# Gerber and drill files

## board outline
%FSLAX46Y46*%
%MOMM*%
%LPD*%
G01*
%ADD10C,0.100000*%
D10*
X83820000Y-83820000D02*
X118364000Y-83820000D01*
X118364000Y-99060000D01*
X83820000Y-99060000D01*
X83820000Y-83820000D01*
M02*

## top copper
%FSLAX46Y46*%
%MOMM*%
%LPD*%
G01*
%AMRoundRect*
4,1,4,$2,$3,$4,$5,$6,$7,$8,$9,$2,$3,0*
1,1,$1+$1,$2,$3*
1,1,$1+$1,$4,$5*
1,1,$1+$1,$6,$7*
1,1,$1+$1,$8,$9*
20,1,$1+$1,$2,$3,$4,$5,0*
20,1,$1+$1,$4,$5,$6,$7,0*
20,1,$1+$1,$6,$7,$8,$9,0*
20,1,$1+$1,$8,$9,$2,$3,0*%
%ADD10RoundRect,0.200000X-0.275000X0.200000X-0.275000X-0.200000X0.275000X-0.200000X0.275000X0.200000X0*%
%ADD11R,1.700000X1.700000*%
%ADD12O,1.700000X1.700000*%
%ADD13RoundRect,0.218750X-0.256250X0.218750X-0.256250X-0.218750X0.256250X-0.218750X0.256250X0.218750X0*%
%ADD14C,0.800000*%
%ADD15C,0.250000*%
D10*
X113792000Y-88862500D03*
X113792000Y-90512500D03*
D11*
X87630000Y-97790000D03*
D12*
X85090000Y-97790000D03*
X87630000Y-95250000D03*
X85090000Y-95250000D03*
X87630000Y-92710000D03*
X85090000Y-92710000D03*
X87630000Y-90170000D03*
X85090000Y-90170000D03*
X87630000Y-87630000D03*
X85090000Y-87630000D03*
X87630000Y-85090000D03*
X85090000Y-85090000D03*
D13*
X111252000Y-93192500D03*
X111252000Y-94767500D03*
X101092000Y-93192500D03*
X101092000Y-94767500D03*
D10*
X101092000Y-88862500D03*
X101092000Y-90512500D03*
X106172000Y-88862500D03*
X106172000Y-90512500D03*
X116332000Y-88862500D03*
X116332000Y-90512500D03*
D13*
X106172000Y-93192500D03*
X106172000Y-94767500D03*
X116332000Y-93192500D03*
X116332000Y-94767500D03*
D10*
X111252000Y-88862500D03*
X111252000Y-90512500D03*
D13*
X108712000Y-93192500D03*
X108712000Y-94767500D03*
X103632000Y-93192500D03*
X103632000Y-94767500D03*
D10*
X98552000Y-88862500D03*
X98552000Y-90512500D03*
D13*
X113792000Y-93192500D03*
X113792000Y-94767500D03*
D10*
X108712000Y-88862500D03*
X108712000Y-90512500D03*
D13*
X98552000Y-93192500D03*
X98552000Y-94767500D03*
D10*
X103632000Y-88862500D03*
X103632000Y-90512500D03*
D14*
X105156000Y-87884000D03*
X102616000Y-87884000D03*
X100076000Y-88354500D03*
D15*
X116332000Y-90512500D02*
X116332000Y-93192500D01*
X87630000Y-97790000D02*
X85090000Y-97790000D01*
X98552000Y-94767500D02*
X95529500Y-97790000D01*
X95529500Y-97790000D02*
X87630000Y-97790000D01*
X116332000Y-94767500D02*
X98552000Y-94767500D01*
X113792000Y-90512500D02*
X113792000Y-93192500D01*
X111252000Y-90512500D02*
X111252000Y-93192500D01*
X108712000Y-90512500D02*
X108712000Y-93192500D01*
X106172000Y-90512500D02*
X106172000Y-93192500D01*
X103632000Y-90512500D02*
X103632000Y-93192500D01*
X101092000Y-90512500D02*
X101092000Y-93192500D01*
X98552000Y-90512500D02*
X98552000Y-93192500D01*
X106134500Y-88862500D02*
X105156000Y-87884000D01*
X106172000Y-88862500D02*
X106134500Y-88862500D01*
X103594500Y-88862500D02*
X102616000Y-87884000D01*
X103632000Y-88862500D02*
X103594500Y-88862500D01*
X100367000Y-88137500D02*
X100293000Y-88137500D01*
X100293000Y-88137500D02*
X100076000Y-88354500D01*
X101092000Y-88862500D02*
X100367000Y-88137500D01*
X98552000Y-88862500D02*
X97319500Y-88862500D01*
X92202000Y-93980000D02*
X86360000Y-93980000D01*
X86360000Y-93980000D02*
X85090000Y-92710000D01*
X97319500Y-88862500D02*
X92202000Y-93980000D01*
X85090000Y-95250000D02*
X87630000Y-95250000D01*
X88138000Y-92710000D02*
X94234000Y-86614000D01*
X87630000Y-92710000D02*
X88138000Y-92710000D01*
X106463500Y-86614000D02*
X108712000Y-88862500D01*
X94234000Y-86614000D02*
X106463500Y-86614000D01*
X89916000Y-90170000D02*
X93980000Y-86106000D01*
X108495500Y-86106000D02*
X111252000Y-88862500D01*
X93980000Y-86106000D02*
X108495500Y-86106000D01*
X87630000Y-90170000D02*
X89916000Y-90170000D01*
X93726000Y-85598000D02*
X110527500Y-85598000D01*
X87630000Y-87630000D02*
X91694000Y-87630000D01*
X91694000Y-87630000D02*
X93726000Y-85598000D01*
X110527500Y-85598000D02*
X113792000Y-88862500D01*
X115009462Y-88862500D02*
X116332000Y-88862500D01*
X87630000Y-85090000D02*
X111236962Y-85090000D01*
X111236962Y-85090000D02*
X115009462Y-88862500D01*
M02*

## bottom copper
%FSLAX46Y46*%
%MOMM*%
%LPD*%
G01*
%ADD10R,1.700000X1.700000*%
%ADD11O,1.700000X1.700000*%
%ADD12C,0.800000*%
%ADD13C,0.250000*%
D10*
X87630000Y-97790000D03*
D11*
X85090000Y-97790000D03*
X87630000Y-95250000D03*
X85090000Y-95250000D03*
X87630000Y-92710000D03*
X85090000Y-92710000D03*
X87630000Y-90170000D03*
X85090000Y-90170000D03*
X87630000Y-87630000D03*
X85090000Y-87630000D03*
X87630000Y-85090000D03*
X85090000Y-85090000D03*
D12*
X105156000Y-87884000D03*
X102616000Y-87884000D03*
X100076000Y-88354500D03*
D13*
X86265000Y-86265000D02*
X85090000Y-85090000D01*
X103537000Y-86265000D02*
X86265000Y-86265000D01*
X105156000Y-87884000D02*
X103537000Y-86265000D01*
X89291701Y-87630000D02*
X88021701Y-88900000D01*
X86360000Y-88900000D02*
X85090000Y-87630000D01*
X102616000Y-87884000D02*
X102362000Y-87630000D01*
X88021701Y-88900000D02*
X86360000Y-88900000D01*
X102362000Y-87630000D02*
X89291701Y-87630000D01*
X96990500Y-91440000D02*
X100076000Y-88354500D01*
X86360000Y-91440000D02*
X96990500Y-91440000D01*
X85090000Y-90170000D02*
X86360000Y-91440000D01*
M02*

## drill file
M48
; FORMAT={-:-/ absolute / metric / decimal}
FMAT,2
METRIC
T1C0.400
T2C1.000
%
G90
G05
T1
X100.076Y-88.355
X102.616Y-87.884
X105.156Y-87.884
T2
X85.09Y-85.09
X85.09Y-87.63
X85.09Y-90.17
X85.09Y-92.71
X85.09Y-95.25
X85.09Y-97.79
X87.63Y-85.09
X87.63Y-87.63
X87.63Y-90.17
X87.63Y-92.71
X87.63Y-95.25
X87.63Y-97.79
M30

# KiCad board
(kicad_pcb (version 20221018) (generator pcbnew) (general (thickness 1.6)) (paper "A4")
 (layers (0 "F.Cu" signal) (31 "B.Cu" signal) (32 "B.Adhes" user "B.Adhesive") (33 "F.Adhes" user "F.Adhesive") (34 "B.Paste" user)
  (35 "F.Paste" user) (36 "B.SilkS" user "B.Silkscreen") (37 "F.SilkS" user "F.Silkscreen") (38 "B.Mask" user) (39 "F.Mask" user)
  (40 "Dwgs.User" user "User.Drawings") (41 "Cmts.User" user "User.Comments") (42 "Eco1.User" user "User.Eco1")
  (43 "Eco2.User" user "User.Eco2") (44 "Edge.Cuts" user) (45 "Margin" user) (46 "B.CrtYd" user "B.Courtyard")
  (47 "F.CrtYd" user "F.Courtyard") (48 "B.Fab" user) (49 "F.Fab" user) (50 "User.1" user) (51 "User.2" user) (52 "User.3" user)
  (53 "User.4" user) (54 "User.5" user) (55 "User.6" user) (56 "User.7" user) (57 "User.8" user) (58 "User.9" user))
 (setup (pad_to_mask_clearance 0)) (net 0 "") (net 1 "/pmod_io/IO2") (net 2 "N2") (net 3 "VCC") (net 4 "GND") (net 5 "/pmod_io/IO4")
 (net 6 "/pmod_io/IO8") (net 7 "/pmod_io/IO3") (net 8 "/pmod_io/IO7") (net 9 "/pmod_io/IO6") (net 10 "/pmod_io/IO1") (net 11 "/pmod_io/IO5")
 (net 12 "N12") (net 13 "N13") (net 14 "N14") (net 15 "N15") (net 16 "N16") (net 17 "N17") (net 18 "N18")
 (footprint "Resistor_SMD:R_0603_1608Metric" (layer "F.Cu") (at 113.792 89.6875 -90)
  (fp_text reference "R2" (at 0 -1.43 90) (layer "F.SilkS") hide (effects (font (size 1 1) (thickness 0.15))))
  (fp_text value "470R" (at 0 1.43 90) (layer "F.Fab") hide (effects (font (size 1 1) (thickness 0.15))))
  (pad "1" smd roundrect (at -0.825 0 270) (size 0.8 0.95) (layers "F.Cu" "F.Paste" "F.Mask") (roundrect_rratio 0.25) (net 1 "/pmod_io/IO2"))
  (pad "2" smd roundrect (at 0.825 0 270) (size 0.8 0.95) (layers "F.Cu" "F.Paste" "F.Mask") (roundrect_rratio 0.25) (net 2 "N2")))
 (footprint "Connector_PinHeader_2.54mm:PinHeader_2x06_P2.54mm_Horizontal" (layer "F.Cu") (at 87.63 97.79 180)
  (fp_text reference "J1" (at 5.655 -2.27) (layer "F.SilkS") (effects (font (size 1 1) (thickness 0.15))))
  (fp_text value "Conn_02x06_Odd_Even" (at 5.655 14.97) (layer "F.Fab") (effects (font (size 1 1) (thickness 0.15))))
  (pad "1" thru_hole rect (at 0 0 180) (size 1.7 1.7) (drill 1) (layers "*.Cu" "*.Mask") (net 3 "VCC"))
  (pad "2" thru_hole oval (at 2.54 0 180) (size 1.7 1.7) (drill 1) (layers "*.Cu" "*.Mask") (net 3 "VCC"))
  (pad "3" thru_hole oval (at 0 2.54 180) (size 1.7 1.7) (drill 1) (layers "*.Cu" "*.Mask") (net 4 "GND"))
  (pad "4" thru_hole oval (at 2.54 2.54 180) (size 1.7 1.7) (drill 1) (layers "*.Cu" "*.Mask") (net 4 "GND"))
  (pad "5" thru_hole oval (at 0 5.08 180) (size 1.7 1.7) (drill 1) (layers "*.Cu" "*.Mask") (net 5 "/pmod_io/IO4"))
  (pad "6" thru_hole oval (at 2.54 5.08 180) (size 1.7 1.7) (drill 1) (layers "*.Cu" "*.Mask") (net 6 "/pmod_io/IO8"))
  (pad "7" thru_hole oval (at 0 7.62 180) (size 1.7 1.7) (drill 1) (layers "*.Cu" "*.Mask") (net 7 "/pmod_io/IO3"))
  (pad "8" thru_hole oval (at 2.54 7.62 180) (size 1.7 1.7) (drill 1) (layers "*.Cu" "*.Mask") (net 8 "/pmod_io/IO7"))
  (pad "9" thru_hole oval (at 0 10.16 180) (size 1.7 1.7) (drill 1) (layers "*.Cu" "*.Mask") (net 1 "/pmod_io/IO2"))
  (pad "10" thru_hole oval (at 2.54 10.16 180) (size 1.7 1.7) (drill 1) (layers "*.Cu" "*.Mask") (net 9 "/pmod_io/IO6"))
  (pad "11" thru_hole oval (at 0 12.7 180) (size 1.7 1.7) (drill 1) (layers "*.Cu" "*.Mask") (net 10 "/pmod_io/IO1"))
  (pad "12" thru_hole oval (at 2.54 12.7 180) (size 1.7 1.7) (drill 1) (layers "*.Cu" "*.Mask") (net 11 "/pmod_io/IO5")))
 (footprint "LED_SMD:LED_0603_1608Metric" (layer "F.Cu") (at 111.252 93.98 -90)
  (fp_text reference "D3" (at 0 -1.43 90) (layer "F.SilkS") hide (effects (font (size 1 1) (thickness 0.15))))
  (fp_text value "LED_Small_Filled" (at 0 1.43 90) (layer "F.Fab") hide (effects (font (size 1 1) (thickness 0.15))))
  (pad "1" smd roundrect (at -0.7875 0 270) (size 0.875 0.95) (layers "F.Cu" "F.Paste" "F.Mask") (roundrect_rratio 0.25) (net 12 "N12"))
  (pad "2" smd roundrect (at 0.7875 0 270) (size 0.875 0.95) (layers "F.Cu" "F.Paste" "F.Mask") (roundrect_rratio 0.25) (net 3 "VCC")))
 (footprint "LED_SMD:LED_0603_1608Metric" (layer "F.Cu") (at 101.092 93.98 -90)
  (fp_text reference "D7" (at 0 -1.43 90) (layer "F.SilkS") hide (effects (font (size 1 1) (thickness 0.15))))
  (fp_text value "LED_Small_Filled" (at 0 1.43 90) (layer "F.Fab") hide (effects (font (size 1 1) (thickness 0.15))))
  (pad "1" smd roundrect (at -0.7875 0 270) (size 0.875 0.95) (layers "F.Cu" "F.Paste" "F.Mask") (roundrect_rratio 0.25) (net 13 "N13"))
  (pad "2" smd roundrect (at 0.7875 0 270) (size 0.875 0.95) (layers "F.Cu" "F.Paste" "F.Mask") (roundrect_rratio 0.25) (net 3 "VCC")))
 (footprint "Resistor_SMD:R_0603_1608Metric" (layer "F.Cu") (at 101.092 89.6875 -90)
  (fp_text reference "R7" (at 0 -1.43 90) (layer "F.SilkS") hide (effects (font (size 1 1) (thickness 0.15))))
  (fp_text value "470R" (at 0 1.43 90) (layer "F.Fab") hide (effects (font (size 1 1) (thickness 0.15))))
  (pad "1" smd roundrect (at -0.825 0 270) (size 0.8 0.95) (layers "F.Cu" "F.Paste" "F.Mask") (roundrect_rratio 0.25) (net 8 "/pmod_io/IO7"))
  (pad "2" smd roundrect (at 0.825 0 270) (size 0.8 0.95) (layers "F.Cu" "F.Paste" "F.Mask") (roundrect_rratio 0.25) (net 13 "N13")))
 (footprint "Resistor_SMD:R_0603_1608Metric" (layer "F.Cu") (at 106.172 89.6875 -90)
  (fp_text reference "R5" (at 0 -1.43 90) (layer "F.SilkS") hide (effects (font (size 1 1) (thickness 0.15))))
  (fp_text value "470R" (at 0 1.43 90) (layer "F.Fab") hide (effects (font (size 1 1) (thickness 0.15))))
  (pad "1" smd roundrect (at -0.825 0 270) (size 0.8 0.95) (layers "F.Cu" "F.Paste" "F.Mask") (roundrect_rratio 0.25)
   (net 11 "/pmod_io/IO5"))
  (pad "2" smd roundrect (at 0.825 0 270) (size 0.8 0.95) (layers "F.Cu" "F.Paste" "F.Mask") (roundrect_rratio 0.25) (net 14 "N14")))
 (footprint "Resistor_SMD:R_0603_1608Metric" (layer "F.Cu") (at 116.332 89.6875 -90)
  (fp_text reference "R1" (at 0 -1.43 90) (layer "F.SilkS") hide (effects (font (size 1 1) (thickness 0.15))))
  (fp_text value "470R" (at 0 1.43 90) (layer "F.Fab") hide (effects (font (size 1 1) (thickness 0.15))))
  (pad "1" smd roundrect (at -0.825 0 270) (size 0.8 0.95) (layers "F.Cu" "F.Paste" "F.Mask") (roundrect_rratio 0.25)
   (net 10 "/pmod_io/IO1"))
  (pad "2" smd roundrect (at 0.825 0 270) (size 0.8 0.95) (layers "F.Cu" "F.Paste" "F.Mask") (roundrect_rratio 0.25) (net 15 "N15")))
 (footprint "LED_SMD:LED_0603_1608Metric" (layer "F.Cu") (at 106.172 93.98 -90)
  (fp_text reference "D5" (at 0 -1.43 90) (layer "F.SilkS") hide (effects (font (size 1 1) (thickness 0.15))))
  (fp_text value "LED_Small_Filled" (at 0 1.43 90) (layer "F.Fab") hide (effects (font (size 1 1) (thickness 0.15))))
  (pad "1" smd roundrect (at -0.7875 0 270) (size 0.875 0.95) (layers "F.Cu" "F.Paste" "F.Mask") (roundrect_rratio 0.25) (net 14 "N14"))
  (pad "2" smd roundrect (at 0.7875 0 270) (size 0.875 0.95) (layers "F.Cu" "F.Paste" "F.Mask") (roundrect_rratio 0.25) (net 3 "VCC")))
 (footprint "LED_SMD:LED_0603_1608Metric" (layer "F.Cu") (at 116.332 93.98 -90)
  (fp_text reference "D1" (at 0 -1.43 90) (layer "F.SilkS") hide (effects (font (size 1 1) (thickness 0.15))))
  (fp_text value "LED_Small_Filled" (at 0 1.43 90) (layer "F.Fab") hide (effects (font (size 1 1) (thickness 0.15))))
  (pad "1" smd roundrect (at -0.7875 0 270) (size 0.875 0.95) (layers "F.Cu" "F.Paste" "F.Mask") (roundrect_rratio 0.25) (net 15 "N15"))
  (pad "2" smd roundrect (at 0.7875 0 270) (size 0.875 0.95) (layers "F.Cu" "F.Paste" "F.Mask") (roundrect_rratio 0.25) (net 3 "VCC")))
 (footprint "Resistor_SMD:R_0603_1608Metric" (layer "F.Cu") (at 111.252 89.6875 -90)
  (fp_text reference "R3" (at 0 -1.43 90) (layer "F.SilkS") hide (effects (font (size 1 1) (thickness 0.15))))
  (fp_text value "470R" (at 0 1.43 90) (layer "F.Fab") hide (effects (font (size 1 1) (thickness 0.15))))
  (pad "1" smd roundrect (at -0.825 0 270) (size 0.8 0.95) (layers "F.Cu" "F.Paste" "F.Mask") (roundrect_rratio 0.25) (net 7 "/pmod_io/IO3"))
  (pad "2" smd roundrect (at 0.825 0 270) (size 0.8 0.95) (layers "F.Cu" "F.Paste" "F.Mask") (roundrect_rratio 0.25) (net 12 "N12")))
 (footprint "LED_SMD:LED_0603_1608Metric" (layer "F.Cu") (at 108.712 93.98 -90)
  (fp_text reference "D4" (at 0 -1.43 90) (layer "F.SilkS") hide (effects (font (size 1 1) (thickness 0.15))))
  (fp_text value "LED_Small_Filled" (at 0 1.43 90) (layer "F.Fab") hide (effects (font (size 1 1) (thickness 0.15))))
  (pad "1" smd roundrect (at -0.7875 0 270) (size 0.875 0.95) (layers "F.Cu" "F.Paste" "F.Mask") (roundrect_rratio 0.25) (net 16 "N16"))
  (pad "2" smd roundrect (at 0.7875 0 270) (size 0.875 0.95) (layers "F.Cu" "F.Paste" "F.Mask") (roundrect_rratio 0.25) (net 3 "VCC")))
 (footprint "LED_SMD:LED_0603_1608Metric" (layer "F.Cu") (at 103.632 93.98 -90)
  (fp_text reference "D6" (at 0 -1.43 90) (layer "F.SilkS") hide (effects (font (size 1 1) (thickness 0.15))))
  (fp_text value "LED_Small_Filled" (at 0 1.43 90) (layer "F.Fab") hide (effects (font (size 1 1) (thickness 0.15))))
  (pad "1" smd roundrect (at -0.7875 0 270) (size 0.875 0.95) (layers "F.Cu" "F.Paste" "F.Mask") (roundrect_rratio 0.25) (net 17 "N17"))
  (pad "2" smd roundrect (at 0.7875 0 270) (size 0.875 0.95) (layers "F.Cu" "F.Paste" "F.Mask") (roundrect_rratio 0.25) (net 3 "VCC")))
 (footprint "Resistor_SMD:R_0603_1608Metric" (layer "F.Cu") (at 98.552 89.6875 -90)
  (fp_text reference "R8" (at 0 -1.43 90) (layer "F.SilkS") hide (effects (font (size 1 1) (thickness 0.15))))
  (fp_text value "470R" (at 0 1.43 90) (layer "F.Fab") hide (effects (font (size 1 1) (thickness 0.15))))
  (pad "1" smd roundrect (at -0.825 0 270) (size 0.8 0.95) (layers "F.Cu" "F.Paste" "F.Mask") (roundrect_rratio 0.25) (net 6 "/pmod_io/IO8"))
  (pad "2" smd roundrect (at 0.825 0 270) (size 0.8 0.95) (layers "F.Cu" "F.Paste" "F.Mask") (roundrect_rratio 0.25) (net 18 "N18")))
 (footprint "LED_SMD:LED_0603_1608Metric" (layer "F.Cu") (at 113.792 93.98 -90)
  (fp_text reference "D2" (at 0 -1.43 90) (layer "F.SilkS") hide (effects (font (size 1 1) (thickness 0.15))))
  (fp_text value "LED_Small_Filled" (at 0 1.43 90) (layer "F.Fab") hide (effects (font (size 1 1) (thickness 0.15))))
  (pad "1" smd roundrect (at -0.7875 0 270) (size 0.875 0.95) (layers "F.Cu" "F.Paste" "F.Mask") (roundrect_rratio 0.25) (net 2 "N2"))
  (pad "2" smd roundrect (at 0.7875 0 270) (size 0.875 0.95) (layers "F.Cu" "F.Paste" "F.Mask") (roundrect_rratio 0.25) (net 3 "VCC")))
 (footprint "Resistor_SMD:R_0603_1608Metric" (layer "F.Cu") (at 108.712 89.6875 -90)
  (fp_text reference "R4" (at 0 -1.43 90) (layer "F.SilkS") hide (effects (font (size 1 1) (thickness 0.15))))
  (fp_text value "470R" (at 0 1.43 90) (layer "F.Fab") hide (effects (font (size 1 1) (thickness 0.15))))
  (pad "1" smd roundrect (at -0.825 0 270) (size 0.8 0.95) (layers "F.Cu" "F.Paste" "F.Mask") (roundrect_rratio 0.25) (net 5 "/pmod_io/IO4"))
  (pad "2" smd roundrect (at 0.825 0 270) (size 0.8 0.95) (layers "F.Cu" "F.Paste" "F.Mask") (roundrect_rratio 0.25) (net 16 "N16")))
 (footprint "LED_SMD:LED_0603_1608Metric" (layer "F.Cu") (at 98.552 93.98 -90)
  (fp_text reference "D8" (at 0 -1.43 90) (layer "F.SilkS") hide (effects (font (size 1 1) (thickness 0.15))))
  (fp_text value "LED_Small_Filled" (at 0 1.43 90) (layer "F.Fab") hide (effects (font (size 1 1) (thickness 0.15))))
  (pad "1" smd roundrect (at -0.7875 0 270) (size 0.875 0.95) (layers "F.Cu" "F.Paste" "F.Mask") (roundrect_rratio 0.25) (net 18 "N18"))
  (pad "2" smd roundrect (at 0.7875 0 270) (size 0.875 0.95) (layers "F.Cu" "F.Paste" "F.Mask") (roundrect_rratio 0.25) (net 3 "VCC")))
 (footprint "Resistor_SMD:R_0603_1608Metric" (layer "F.Cu") (at 103.632 89.6875 -90)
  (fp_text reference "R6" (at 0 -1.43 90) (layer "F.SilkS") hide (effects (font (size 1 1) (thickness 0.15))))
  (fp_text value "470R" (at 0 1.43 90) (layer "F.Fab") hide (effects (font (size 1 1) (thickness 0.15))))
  (pad "1" smd roundrect (at -0.825 0 270) (size 0.8 0.95) (layers "F.Cu" "F.Paste" "F.Mask") (roundrect_rratio 0.25) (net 9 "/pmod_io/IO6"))
  (pad "2" smd roundrect (at 0.825 0 270) (size 0.8 0.95) (layers "F.Cu" "F.Paste" "F.Mask") (roundrect_rratio 0.25) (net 17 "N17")))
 (gr_rect (start 83.82 83.82) (end 118.364 99.06) (stroke (width 0.1) (type default)) (fill none) (layer "Edge.Cuts"))
 (segment (start 116.332 90.5125) (end 116.332 93.1925) (width 0.25) (layer "F.Cu") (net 15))
 (segment (start 87.63 97.79) (end 85.09 97.79) (width 0.25) (layer "F.Cu") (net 3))
 (segment (start 98.552 94.7675) (end 95.5295 97.79) (width 0.25) (layer "F.Cu") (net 3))
 (segment (start 95.5295 97.79) (end 87.63 97.79) (width 0.25) (layer "F.Cu") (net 3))
 (segment (start 116.332 94.7675) (end 98.552 94.7675) (width 0.25) (layer "F.Cu") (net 3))
 (segment (start 113.792 90.5125) (end 113.792 93.1925) (width 0.25) (layer "F.Cu") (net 2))
 (segment (start 111.252 90.5125) (end 111.252 93.1925) (width 0.25) (layer "F.Cu") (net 12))
 (segment (start 108.712 90.5125) (end 108.712 93.1925) (width 0.25) (layer "F.Cu") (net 16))
 (segment (start 106.172 90.5125) (end 106.172 93.1925) (width 0.25) (layer "F.Cu") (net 14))
 (segment (start 103.632 90.5125) (end 103.632 93.1925) (width 0.25) (layer "F.Cu") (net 17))
 (segment (start 101.092 90.5125) (end 101.092 93.1925) (width 0.25) (layer "F.Cu") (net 13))
 (segment (start 98.552 90.5125) (end 98.552 93.1925) (width 0.25) (layer "F.Cu") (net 18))
 (segment (start 106.1345 88.8625) (end 105.156 87.884) (width 0.25) (layer "F.Cu") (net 11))
 (segment (start 106.172 88.8625) (end 106.1345 88.8625) (width 0.25) (layer "F.Cu") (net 11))
 (via (at 105.156 87.884) (size 0.8) (drill 0.4) (layers "F.Cu" "B.Cu") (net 11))
 (segment (start 86.265 86.265) (end 85.09 85.09) (width 0.25) (layer "B.Cu") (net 11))
 (segment (start 103.537 86.265) (end 86.265 86.265) (width 0.25) (layer "B.Cu") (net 11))
 (segment (start 105.156 87.884) (end 103.537 86.265) (width 0.25) (layer "B.Cu") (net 11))
 (segment (start 103.5945 88.8625) (end 102.616 87.884) (width 0.25) (layer "F.Cu") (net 9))
 (segment (start 103.632 88.8625) (end 103.5945 88.8625) (width 0.25) (layer "F.Cu") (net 9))
 (via (at 102.616 87.884) (size 0.8) (drill 0.4) (layers "F.Cu" "B.Cu") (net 9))
 (segment (start 89.291701 87.63) (end 88.021701 88.9) (width 0.25) (layer "B.Cu") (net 9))
 (segment (start 86.36 88.9) (end 85.09 87.63) (width 0.25) (layer "B.Cu") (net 9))
 (segment (start 102.616 87.884) (end 102.362 87.63) (width 0.25) (layer "B.Cu") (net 9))
 (segment (start 88.021701 88.9) (end 86.36 88.9) (width 0.25) (layer "B.Cu") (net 9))
 (segment (start 102.362 87.63) (end 89.291701 87.63) (width 0.25) (layer "B.Cu") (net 9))
 (segment (start 100.367 88.1375) (end 100.293 88.1375) (width 0.25) (layer "F.Cu") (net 8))
 (segment (start 100.293 88.1375) (end 100.076 88.3545) (width 0.25) (layer "F.Cu") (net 8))
 (segment (start 101.092 88.8625) (end 100.367 88.1375) (width 0.25) (layer "F.Cu") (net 8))
 (via (at 100.076 88.3545) (size 0.8) (drill 0.4) (layers "F.Cu" "B.Cu") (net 8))
 (segment (start 96.9905 91.44) (end 100.076 88.3545) (width 0.25) (layer "B.Cu") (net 8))
 (segment (start 86.36 91.44) (end 96.9905 91.44) (width 0.25) (layer "B.Cu") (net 8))
 (segment (start 85.09 90.17) (end 86.36 91.44) (width 0.25) (layer "B.Cu") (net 8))
 (segment (start 98.552 88.8625) (end 97.3195 88.8625) (width 0.25) (layer "F.Cu") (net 6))
 (segment (start 92.202 93.98) (end 86.36 93.98) (width 0.25) (layer "F.Cu") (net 6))
 (segment (start 86.36 93.98) (end 85.09 92.71) (width 0.25) (layer "F.Cu") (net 6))
 (segment (start 97.3195 88.8625) (end 92.202 93.98) (width 0.25) (layer "F.Cu") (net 6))
 (segment (start 85.09 95.25) (end 87.63 95.25) (width 0.25) (layer "F.Cu") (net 4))
 (segment (start 88.138 92.71) (end 94.234 86.614) (width 0.25) (layer "F.Cu") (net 5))
 (segment (start 87.63 92.71) (end 88.138 92.71) (width 0.25) (layer "F.Cu") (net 5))
 (segment (start 106.4635 86.614) (end 108.712 88.8625) (width 0.25) (layer "F.Cu") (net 5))
 (segment (start 94.234 86.614) (end 106.4635 86.614) (width 0.25) (layer "F.Cu") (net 5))
 (segment (start 89.916 90.17) (end 93.98 86.106) (width 0.25) (layer "F.Cu") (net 7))
 (segment (start 108.4955 86.106) (end 111.252 88.8625) (width 0.25) (layer "F.Cu") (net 7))
 (segment (start 93.98 86.106) (end 108.4955 86.106) (width 0.25) (layer "F.Cu") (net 7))
 (segment (start 87.63 90.17) (end 89.916 90.17) (width 0.25) (layer "F.Cu") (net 7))
 (segment (start 93.726 85.598) (end 110.5275 85.598) (width 0.25) (layer "F.Cu") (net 1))
 (segment (start 87.63 87.63) (end 91.694 87.63) (width 0.25) (layer "F.Cu") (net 1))
 (segment (start 91.694 87.63) (end 93.726 85.598) (width 0.25) (layer "F.Cu") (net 1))
 (segment (start 110.5275 85.598) (end 113.792 88.8625) (width 0.25) (layer "F.Cu") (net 1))
 (segment (start 115.009462 88.8625) (end 116.332 88.8625) (width 0.25) (layer "F.Cu") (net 10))
 (segment (start 87.63 85.09) (end 111.236962 85.09) (width 0.25) (layer "F.Cu") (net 10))
 (segment (start 111.236962 85.09) (end 115.009462 88.8625) (width 0.25) (layer "F.Cu") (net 10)))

